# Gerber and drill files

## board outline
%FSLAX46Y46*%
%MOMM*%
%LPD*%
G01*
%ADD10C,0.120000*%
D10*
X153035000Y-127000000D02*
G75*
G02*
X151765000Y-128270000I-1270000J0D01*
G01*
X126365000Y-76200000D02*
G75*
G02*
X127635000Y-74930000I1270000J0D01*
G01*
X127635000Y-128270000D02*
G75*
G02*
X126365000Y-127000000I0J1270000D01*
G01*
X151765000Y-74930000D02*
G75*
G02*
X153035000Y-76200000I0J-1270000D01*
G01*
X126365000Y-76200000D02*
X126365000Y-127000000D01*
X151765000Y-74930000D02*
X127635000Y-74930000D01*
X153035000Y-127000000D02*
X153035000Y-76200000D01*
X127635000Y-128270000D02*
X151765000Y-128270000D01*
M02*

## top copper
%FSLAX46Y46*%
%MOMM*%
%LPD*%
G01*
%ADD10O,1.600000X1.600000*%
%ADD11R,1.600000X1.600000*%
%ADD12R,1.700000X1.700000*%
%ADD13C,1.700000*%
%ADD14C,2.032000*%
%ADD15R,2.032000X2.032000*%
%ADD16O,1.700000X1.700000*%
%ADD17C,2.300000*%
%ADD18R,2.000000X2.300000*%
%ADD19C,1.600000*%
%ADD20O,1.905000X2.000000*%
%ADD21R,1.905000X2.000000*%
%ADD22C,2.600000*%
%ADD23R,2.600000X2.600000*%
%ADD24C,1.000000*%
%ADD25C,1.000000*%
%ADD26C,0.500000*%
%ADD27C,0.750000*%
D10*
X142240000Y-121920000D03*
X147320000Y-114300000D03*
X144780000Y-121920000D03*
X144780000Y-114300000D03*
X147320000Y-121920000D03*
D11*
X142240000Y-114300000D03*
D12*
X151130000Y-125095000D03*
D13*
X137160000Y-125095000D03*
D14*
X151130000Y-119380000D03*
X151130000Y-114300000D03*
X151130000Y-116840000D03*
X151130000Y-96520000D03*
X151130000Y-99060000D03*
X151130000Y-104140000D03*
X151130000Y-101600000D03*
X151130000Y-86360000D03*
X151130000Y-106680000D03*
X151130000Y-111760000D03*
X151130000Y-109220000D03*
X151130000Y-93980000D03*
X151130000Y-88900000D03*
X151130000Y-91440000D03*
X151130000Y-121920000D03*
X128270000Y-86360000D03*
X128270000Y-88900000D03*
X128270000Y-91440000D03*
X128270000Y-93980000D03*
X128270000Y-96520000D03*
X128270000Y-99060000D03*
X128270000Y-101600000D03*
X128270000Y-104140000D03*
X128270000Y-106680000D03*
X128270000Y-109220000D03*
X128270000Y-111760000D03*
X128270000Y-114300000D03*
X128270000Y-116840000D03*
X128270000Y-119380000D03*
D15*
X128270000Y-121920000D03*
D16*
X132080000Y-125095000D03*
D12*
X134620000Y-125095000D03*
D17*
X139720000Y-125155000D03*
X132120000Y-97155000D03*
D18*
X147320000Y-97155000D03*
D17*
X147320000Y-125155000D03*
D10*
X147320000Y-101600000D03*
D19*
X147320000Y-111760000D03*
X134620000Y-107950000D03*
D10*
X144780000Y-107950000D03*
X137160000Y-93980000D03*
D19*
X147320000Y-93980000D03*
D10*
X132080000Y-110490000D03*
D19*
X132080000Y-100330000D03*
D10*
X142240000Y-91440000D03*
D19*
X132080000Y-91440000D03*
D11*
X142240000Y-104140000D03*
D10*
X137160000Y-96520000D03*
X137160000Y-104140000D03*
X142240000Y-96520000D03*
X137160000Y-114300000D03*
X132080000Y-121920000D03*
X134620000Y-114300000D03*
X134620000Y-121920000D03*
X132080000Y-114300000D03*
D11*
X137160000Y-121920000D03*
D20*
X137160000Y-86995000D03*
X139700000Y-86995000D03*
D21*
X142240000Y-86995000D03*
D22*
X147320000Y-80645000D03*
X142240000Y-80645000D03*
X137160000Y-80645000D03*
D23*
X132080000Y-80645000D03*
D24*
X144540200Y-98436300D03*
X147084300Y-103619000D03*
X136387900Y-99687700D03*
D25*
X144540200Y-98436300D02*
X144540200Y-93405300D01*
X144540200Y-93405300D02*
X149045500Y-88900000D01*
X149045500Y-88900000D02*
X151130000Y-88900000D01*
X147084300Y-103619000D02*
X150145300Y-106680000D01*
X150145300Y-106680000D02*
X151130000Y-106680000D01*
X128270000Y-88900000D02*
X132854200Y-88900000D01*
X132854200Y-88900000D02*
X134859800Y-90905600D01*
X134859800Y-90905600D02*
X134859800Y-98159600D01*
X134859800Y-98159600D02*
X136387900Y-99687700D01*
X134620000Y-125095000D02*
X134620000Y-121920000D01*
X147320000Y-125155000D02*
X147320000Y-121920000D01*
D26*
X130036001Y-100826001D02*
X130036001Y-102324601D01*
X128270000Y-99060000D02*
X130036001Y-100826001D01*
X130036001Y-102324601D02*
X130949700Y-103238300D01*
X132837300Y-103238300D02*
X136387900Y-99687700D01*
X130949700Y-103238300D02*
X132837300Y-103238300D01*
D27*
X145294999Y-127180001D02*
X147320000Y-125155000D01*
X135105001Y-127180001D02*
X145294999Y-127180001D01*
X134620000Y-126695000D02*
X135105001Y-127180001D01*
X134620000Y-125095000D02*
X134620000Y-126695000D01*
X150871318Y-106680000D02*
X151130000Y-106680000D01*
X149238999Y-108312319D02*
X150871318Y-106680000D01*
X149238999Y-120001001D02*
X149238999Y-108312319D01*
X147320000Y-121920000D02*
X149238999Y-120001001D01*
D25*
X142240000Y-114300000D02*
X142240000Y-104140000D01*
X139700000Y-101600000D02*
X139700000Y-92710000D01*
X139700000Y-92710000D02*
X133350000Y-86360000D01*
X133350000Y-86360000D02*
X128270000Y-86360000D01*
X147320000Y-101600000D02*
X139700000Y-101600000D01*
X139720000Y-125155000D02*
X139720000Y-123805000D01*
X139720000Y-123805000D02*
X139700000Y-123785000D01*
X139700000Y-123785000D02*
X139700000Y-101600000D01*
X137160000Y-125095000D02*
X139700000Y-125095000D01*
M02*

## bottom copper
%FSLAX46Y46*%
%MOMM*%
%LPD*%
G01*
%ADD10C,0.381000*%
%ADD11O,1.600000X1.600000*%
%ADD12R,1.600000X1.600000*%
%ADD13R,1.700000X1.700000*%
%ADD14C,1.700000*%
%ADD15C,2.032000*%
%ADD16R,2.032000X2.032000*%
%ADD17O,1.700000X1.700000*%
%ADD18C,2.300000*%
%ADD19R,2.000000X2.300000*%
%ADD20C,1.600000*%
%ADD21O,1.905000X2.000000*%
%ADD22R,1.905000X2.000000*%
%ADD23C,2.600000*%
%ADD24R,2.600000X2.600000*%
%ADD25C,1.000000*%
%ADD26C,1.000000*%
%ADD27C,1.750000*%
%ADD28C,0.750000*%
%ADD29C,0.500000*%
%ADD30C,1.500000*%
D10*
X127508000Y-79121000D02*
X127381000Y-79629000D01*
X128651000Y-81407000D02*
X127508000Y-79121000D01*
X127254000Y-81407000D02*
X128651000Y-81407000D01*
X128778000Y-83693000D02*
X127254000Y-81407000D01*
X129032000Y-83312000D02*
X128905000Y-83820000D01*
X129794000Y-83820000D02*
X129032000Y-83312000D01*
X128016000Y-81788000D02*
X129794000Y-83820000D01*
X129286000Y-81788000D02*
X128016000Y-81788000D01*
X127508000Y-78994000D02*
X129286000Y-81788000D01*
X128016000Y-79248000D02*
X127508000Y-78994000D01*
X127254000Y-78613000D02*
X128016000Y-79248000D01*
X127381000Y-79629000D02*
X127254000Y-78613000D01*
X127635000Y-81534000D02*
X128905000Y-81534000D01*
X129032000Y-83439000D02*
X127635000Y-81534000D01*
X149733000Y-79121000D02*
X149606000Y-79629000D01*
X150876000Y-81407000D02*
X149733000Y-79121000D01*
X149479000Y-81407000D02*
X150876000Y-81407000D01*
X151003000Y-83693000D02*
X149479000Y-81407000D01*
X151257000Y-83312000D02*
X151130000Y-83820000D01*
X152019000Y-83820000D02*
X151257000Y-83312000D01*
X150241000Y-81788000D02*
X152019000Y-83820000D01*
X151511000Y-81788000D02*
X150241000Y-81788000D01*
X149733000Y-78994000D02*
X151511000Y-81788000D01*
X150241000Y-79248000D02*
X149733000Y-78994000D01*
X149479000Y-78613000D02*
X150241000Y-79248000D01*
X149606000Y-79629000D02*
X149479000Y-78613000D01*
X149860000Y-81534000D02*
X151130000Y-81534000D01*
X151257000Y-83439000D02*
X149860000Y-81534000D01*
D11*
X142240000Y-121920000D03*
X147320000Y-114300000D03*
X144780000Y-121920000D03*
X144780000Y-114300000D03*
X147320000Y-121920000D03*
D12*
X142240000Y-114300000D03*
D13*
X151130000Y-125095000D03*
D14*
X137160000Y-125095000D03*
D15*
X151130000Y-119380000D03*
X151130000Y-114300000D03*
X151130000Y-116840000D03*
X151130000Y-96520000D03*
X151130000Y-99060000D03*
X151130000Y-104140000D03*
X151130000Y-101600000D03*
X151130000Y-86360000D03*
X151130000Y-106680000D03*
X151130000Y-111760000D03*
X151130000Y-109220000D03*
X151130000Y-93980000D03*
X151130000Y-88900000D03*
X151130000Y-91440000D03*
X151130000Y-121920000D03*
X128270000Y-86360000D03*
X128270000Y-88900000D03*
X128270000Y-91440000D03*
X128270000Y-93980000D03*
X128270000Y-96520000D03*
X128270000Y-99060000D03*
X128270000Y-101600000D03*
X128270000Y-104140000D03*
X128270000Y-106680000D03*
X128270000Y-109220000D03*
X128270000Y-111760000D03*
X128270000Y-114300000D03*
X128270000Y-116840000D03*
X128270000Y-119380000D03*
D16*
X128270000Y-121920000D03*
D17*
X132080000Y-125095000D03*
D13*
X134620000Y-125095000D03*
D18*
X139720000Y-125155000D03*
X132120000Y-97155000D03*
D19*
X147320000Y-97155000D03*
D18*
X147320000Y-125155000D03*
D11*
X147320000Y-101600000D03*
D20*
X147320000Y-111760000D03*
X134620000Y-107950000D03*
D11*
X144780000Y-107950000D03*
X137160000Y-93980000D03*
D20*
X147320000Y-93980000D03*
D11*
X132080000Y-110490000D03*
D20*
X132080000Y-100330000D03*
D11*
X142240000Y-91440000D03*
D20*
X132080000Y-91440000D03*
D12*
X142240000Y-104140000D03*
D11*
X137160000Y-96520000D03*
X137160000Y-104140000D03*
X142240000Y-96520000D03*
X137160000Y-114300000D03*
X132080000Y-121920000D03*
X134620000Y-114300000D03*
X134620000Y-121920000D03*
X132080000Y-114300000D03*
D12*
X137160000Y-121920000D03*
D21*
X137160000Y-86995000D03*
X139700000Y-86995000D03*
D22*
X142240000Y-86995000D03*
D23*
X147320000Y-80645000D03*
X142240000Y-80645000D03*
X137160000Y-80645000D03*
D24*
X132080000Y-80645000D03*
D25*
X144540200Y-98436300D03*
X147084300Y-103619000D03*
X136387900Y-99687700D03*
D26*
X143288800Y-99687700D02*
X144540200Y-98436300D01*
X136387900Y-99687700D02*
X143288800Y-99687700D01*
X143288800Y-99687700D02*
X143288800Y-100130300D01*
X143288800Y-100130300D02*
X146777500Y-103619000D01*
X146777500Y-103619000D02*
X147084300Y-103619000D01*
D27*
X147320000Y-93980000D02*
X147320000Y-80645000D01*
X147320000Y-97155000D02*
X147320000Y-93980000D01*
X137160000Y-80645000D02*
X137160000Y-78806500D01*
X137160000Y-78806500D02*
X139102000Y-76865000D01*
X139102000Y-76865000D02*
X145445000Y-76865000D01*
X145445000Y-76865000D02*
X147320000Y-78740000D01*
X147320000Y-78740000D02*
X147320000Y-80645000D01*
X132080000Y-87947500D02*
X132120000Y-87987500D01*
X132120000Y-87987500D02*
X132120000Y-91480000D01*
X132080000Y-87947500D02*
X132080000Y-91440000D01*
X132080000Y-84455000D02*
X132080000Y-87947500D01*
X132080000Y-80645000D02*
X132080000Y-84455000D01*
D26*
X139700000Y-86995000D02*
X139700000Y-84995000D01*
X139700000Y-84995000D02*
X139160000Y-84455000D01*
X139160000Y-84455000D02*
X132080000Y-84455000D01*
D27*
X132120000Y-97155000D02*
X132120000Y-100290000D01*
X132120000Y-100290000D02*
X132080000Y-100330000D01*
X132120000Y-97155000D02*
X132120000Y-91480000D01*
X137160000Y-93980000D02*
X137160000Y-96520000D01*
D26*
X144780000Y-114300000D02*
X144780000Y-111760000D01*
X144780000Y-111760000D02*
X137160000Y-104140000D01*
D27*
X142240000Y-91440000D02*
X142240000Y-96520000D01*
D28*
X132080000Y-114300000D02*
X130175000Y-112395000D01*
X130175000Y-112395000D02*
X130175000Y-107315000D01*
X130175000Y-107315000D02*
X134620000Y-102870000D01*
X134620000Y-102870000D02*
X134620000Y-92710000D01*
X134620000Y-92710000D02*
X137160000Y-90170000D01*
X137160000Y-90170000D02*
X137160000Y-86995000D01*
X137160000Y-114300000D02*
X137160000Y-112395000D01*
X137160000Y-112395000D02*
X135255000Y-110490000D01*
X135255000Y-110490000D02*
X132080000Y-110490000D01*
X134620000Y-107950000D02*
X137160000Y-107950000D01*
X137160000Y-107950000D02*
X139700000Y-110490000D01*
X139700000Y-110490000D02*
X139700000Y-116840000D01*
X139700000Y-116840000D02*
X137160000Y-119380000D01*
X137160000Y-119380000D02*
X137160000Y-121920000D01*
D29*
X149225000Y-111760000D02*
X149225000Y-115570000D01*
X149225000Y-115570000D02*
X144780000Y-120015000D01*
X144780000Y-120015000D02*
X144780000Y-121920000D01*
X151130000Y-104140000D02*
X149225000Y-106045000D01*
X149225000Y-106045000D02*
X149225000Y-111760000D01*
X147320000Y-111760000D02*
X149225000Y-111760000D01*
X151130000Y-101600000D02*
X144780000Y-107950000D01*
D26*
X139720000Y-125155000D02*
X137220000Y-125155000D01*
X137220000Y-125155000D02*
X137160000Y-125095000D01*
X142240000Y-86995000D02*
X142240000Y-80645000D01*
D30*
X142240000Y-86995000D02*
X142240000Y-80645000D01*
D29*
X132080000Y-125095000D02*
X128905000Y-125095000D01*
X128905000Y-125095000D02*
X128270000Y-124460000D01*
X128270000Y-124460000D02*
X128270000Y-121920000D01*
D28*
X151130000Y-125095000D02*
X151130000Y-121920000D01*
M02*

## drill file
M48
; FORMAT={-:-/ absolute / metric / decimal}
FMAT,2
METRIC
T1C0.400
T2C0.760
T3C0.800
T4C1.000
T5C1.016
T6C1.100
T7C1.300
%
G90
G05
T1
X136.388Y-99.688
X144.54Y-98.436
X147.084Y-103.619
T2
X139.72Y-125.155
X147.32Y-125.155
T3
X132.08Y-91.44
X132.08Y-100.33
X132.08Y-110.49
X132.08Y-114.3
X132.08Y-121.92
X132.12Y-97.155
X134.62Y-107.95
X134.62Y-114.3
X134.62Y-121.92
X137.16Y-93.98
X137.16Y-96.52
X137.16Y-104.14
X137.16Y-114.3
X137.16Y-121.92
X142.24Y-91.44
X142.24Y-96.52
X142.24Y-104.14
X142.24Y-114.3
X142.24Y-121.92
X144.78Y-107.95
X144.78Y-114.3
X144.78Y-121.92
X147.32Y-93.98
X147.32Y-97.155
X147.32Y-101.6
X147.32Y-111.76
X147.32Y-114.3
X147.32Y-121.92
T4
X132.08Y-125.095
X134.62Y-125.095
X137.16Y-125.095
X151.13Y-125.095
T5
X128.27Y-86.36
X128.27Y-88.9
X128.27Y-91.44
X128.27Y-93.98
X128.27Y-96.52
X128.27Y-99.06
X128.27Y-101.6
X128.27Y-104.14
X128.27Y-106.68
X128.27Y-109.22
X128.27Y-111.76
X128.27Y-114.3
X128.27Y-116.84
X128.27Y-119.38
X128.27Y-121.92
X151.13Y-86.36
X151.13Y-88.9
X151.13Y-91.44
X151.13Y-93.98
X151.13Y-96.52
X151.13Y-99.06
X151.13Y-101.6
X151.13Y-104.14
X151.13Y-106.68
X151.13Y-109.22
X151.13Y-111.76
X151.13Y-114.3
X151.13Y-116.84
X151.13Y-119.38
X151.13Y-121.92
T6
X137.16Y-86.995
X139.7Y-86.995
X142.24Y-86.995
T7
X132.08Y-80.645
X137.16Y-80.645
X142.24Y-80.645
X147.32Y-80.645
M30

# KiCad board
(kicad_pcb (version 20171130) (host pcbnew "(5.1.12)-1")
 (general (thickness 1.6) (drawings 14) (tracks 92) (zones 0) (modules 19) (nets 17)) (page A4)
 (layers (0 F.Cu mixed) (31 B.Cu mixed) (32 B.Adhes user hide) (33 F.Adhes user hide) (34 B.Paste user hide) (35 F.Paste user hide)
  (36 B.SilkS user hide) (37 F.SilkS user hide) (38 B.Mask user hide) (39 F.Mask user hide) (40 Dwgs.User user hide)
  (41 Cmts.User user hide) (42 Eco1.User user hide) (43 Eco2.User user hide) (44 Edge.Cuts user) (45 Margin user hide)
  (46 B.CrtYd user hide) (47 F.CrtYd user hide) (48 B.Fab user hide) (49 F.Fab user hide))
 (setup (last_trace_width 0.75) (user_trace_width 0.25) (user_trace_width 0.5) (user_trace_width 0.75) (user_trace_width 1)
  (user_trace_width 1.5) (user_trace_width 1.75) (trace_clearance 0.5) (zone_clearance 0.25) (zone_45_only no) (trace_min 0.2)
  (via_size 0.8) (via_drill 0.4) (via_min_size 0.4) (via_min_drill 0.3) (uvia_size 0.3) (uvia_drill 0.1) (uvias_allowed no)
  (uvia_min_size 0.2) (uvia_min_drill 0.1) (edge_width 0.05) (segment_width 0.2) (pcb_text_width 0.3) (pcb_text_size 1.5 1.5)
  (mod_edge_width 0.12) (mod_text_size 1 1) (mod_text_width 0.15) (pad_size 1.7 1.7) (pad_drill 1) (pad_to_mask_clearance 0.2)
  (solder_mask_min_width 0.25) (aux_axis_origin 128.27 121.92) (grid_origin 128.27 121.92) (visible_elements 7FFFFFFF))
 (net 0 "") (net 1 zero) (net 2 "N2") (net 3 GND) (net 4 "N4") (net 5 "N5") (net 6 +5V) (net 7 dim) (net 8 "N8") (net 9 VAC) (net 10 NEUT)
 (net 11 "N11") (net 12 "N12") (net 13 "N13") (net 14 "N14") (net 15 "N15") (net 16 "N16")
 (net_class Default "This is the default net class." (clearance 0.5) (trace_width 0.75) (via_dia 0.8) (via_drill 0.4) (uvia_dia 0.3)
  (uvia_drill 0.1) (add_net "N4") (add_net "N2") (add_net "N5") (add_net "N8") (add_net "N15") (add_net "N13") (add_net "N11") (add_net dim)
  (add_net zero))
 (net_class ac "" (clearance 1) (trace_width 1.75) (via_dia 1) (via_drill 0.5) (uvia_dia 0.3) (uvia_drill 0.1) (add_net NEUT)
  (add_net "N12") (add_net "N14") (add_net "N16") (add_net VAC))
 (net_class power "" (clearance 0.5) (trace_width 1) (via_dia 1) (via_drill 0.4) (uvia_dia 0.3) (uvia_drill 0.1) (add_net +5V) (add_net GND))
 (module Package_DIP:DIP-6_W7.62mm (layer B.Cu) (at 142.24 114.3 270)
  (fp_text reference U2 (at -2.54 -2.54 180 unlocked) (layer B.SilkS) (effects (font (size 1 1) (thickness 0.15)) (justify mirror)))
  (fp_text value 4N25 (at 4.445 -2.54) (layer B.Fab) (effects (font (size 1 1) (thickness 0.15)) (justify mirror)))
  (pad 6 thru_hole oval (at 7.62 0 270) (size 1.6 1.6) (drill 0.8) (layers *.Cu *.Mask))
  (pad 3 thru_hole oval (at 0 -5.08 270) (size 1.6 1.6) (drill 0.8) (layers *.Cu *.Mask))
  (pad 5 thru_hole oval (at 7.62 -2.54 270) (size 1.6 1.6) (drill 0.8) (layers *.Cu *.Mask) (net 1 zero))
  (pad 2 thru_hole oval (at 0 -2.54 270) (size 1.6 1.6) (drill 0.8) (layers *.Cu *.Mask) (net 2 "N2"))
  (pad 4 thru_hole oval (at 7.62 -5.08 270) (size 1.6 1.6) (drill 0.8) (layers *.Cu *.Mask) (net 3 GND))
  (pad 1 thru_hole rect (at 0 0 270) (size 1.6 1.6) (drill 0.8) (layers *.Cu *.Mask) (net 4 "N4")))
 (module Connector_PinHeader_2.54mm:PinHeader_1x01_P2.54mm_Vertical (layer B.Cu) (at 151.13 125.095)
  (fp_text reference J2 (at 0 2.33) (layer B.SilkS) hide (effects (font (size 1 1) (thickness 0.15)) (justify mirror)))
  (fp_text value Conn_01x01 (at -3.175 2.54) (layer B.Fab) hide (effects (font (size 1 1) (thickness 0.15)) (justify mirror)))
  (pad 1 thru_hole rect (at 0 0) (size 1.7 1.7) (drill 1) (layers *.Cu *.Mask) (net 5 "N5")))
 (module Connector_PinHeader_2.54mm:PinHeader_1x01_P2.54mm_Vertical (layer B.Cu) (at 137.16 125.095)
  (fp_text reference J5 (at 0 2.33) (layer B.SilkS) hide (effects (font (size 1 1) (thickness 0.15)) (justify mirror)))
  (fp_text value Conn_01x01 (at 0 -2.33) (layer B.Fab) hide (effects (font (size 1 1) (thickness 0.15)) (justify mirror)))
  (pad 1 thru_hole circle (at 0 0) (size 1.7 1.7) (drill 1) (layers *.Cu *.Mask) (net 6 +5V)))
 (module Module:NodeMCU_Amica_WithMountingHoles (layer B.Cu) (at 128.27 121.92)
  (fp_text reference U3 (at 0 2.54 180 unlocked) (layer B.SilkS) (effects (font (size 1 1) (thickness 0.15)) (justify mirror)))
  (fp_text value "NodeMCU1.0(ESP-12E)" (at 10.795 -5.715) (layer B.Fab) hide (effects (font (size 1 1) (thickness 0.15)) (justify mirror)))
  (pad 29 thru_hole circle (at 22.86 -2.54) (size 2.032 2.032) (drill 1.016) (layers *.Cu *.Mask))
  (pad 27 thru_hole circle (at 22.86 -7.62) (size 2.032 2.032) (drill 1.016) (layers *.Cu *.Mask))
  (pad 28 thru_hole circle (at 22.86 -5.08) (size 2.032 2.032) (drill 1.016) (layers *.Cu *.Mask))
  (pad 20 thru_hole circle (at 22.86 -25.4) (size 2.032 2.032) (drill 1.016) (layers *.Cu *.Mask))
  (pad 21 thru_hole circle (at 22.86 -22.86) (size 2.032 2.032) (drill 1.016) (layers *.Cu *.Mask))
  (pad 23 thru_hole circle (at 22.86 -17.78) (size 2.032 2.032) (drill 1.016) (layers *.Cu *.Mask) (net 1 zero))
  (pad 22 thru_hole circle (at 22.86 -20.32) (size 2.032 2.032) (drill 1.016) (layers *.Cu *.Mask) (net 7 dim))
  (pad 16 thru_hole circle (at 22.86 -35.56) (size 2.032 2.032) (drill 1.016) (layers *.Cu *.Mask))
  (pad 24 thru_hole circle (at 22.86 -15.24) (size 2.032 2.032) (drill 1.016) (layers *.Cu *.Mask) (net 3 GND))
  (pad 26 thru_hole circle (at 22.86 -10.16) (size 2.032 2.032) (drill 1.016) (layers *.Cu *.Mask))
  (pad 25 thru_hole circle (at 22.86 -12.7) (size 2.032 2.032) (drill 1.016) (layers *.Cu *.Mask))
  (pad 19 thru_hole circle (at 22.86 -27.94) (size 2.032 2.032) (drill 1.016) (layers *.Cu *.Mask))
  (pad 17 thru_hole circle (at 22.86 -33.02) (size 2.032 2.032) (drill 1.016) (layers *.Cu *.Mask) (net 3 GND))
  (pad 18 thru_hole circle (at 22.86 -30.48) (size 2.032 2.032) (drill 1.016) (layers *.Cu *.Mask))
  (pad 30 thru_hole circle (at 22.86 0) (size 2.032 2.032) (drill 1.016) (layers *.Cu *.Mask) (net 5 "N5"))
  (pad 15 thru_hole circle (at 0 -35.56) (size 2.032 2.032) (drill 1.016) (layers *.Cu *.Mask) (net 6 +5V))
  (pad 14 thru_hole circle (at 0 -33.02) (size 2.032 2.032) (drill 1.016) (layers *.Cu *.Mask) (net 3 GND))
  (pad 13 thru_hole circle (at 0 -30.48) (size 2.032 2.032) (drill 1.016) (layers *.Cu *.Mask))
  (pad 12 thru_hole circle (at 0 -27.94) (size 2.032 2.032) (drill 1.016) (layers *.Cu *.Mask))
  (pad 11 thru_hole circle (at 0 -25.4) (size 2.032 2.032) (drill 1.016) (layers *.Cu *.Mask))
  (pad 10 thru_hole circle (at 0 -22.86) (size 2.032 2.032) (drill 1.016) (layers *.Cu *.Mask) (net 3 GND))
  (pad 9 thru_hole circle (at 0 -20.32) (size 2.032 2.032) (drill 1.016) (layers *.Cu *.Mask))
  (pad 8 thru_hole circle (at 0 -17.78) (size 2.032 2.032) (drill 1.016) (layers *.Cu *.Mask))
  (pad 7 thru_hole circle (at 0 -15.24) (size 2.032 2.032) (drill 1.016) (layers *.Cu *.Mask))
  (pad 6 thru_hole circle (at 0 -12.7) (size 2.032 2.032) (drill 1.016) (layers *.Cu *.Mask))
  (pad 5 thru_hole circle (at 0 -10.16) (size 2.032 2.032) (drill 1.016) (layers *.Cu *.Mask))
  (pad 4 thru_hole circle (at 0 -7.62) (size 2.032 2.032) (drill 1.016) (layers *.Cu *.Mask))
  (pad 3 thru_hole circle (at 0 -5.08) (size 2.032 2.032) (drill 1.016) (layers *.Cu *.Mask))
  (pad 2 thru_hole circle (at 0 -2.54) (size 2.032 2.032) (drill 1.016) (layers *.Cu *.Mask))
  (pad 1 thru_hole rect (at 0 0) (size 2.032 2.032) (drill 1.016) (layers *.Cu *.Mask) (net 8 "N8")))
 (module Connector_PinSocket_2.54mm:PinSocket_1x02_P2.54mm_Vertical (layer B.Cu) (at 134.62 125.095 90)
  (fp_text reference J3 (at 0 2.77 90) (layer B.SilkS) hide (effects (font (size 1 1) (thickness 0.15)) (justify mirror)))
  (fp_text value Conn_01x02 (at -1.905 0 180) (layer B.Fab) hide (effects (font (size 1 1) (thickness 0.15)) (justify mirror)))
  (pad 2 thru_hole oval (at 0 -2.54 90) (size 1.7 1.7) (drill 1) (layers *.Cu *.Mask) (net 8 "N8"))
  (pad 1 thru_hole rect (at 0 0 90) (size 1.7 1.7) (drill 1) (layers *.Cu *.Mask) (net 3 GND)))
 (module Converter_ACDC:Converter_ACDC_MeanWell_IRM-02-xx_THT (layer F.Cu) (at 147.32 97.155 270)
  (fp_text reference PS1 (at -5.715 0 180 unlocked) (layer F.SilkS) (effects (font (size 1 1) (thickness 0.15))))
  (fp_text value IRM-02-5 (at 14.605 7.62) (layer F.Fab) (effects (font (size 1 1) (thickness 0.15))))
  (pad 4 thru_hole circle (at 28 7.6 270) (size 2.3 2.3) (drill 0.76) (layers *.Cu *.Mask) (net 6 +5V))
  (pad 2 thru_hole circle (at 0 15.2 270) (size 2.3 2.3) (drill 0.8) (layers *.Cu *.Mask) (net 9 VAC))
  (pad 1 thru_hole rect (at 0 0 270) (size 2.3 2) (drill 0.8) (layers *.Cu *.Mask) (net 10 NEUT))
  (pad 3 thru_hole circle (at 28 0 270) (size 2.3 2.3) (drill 0.76) (layers *.Cu *.Mask) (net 3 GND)))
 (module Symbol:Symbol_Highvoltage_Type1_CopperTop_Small (layer B.Cu) (at 127.635 80.645)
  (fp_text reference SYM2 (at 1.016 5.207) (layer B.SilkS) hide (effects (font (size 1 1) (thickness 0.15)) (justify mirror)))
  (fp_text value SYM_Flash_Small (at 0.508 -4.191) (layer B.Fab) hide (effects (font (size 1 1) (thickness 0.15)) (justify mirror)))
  (fp_line (start -0.127 -1.524) (end -0.254 -1.016) (layer B.Cu) (width 0.381))
  (fp_line (start 1.016 0.762) (end -0.127 -1.524) (layer B.Cu) (width 0.381))
  (fp_line (start -0.381 0.762) (end 1.016 0.762) (layer B.Cu) (width 0.381))
  (fp_line (start 1.143 3.048) (end -0.381 0.762) (layer B.Cu) (width 0.381))
  (fp_line (start 1.397 2.667) (end 1.27 3.175) (layer B.Cu) (width 0.381))
  (fp_line (start 2.159 3.175) (end 1.397 2.667) (layer B.Cu) (width 0.381))
  (fp_line (start 0.381 1.143) (end 2.159 3.175) (layer B.Cu) (width 0.381))
  (fp_line (start 1.651 1.143) (end 0.381 1.143) (layer B.Cu) (width 0.381))
  (fp_line (start -0.127 -1.651) (end 1.651 1.143) (layer B.Cu) (width 0.381))
  (fp_line (start 0.381 -1.397) (end -0.127 -1.651) (layer B.Cu) (width 0.381))
  (fp_line (start -0.381 -2.032) (end 0.381 -1.397) (layer B.Cu) (width 0.381))
  (fp_line (start -0.254 -1.016) (end -0.381 -2.032) (layer B.Cu) (width 0.381))
  (fp_line (start 0 0.889) (end 1.27 0.889) (layer B.Cu) (width 0.381))
  (fp_line (start 1.397 2.794) (end 0 0.889) (layer B.Cu) (width 0.381)))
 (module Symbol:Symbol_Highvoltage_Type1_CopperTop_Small (layer B.Cu) (at 149.86 80.645)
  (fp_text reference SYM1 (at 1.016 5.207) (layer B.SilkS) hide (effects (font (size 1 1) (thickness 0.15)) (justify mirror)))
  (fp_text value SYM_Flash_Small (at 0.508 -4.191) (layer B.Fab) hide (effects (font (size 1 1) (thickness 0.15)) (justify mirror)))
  (fp_line (start -0.127 -1.524) (end -0.254 -1.016) (layer B.Cu) (width 0.381))
  (fp_line (start 1.016 0.762) (end -0.127 -1.524) (layer B.Cu) (width 0.381))
  (fp_line (start -0.381 0.762) (end 1.016 0.762) (layer B.Cu) (width 0.381))
  (fp_line (start 1.143 3.048) (end -0.381 0.762) (layer B.Cu) (width 0.381))
  (fp_line (start 1.397 2.667) (end 1.27 3.175) (layer B.Cu) (width 0.381))
  (fp_line (start 2.159 3.175) (end 1.397 2.667) (layer B.Cu) (width 0.381))
  (fp_line (start 0.381 1.143) (end 2.159 3.175) (layer B.Cu) (width 0.381))
  (fp_line (start 1.651 1.143) (end 0.381 1.143) (layer B.Cu) (width 0.381))
  (fp_line (start -0.127 -1.651) (end 1.651 1.143) (layer B.Cu) (width 0.381))
  (fp_line (start 0.381 -1.397) (end -0.127 -1.651) (layer B.Cu) (width 0.381))
  (fp_line (start -0.381 -2.032) (end 0.381 -1.397) (layer B.Cu) (width 0.381))
  (fp_line (start -0.254 -1.016) (end -0.381 -2.032) (layer B.Cu) (width 0.381))
  (fp_line (start 0 0.889) (end 1.27 0.889) (layer B.Cu) (width 0.381))
  (fp_line (start 1.397 2.794) (end 0 0.889) (layer B.Cu) (width 0.381)))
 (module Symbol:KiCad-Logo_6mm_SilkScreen (layer F.Cu) (at 143.51 105.41 90)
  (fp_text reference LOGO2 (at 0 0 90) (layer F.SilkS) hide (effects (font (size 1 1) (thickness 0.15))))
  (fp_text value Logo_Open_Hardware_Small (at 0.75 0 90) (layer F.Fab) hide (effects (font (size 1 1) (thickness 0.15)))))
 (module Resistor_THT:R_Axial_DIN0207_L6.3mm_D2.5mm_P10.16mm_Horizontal (layer B.Cu) (at 147.32 111.76 90)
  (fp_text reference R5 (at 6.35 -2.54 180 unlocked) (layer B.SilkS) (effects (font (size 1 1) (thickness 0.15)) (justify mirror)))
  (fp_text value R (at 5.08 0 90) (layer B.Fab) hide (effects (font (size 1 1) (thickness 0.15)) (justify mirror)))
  (pad 2 thru_hole oval (at 10.16 0 90) (size 1.6 1.6) (drill 0.8) (layers *.Cu *.Mask) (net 6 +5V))
  (pad 1 thru_hole circle (at 0 0 90) (size 1.6 1.6) (drill 0.8) (layers *.Cu *.Mask) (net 1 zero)))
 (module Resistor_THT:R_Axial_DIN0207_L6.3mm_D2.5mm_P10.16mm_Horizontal (layer B.Cu) (at 134.62 107.95)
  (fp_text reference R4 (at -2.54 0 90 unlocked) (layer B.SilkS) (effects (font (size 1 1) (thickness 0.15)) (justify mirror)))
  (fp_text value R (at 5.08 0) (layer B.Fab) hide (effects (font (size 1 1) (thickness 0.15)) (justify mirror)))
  (pad 1 thru_hole circle (at 0 0) (size 1.6 1.6) (drill 0.8) (layers *.Cu *.Mask) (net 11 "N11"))
  (pad 2 thru_hole oval (at 10.16 0) (size 1.6 1.6) (drill 0.8) (layers *.Cu *.Mask) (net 7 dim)))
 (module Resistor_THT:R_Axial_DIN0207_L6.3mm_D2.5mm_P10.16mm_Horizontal (layer B.Cu) (at 147.32 93.98 180)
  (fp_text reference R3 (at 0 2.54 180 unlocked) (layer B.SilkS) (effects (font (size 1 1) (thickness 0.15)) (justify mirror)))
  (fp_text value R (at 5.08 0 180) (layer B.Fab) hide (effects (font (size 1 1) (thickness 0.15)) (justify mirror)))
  (pad 2 thru_hole oval (at 10.16 0 180) (size 1.6 1.6) (drill 0.8) (layers *.Cu *.Mask) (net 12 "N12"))
  (pad 1 thru_hole circle (at 0 0 180) (size 1.6 1.6) (drill 0.8) (layers *.Cu *.Mask) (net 10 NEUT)))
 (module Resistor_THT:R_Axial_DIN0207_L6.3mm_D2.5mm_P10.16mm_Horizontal (layer B.Cu) (at 132.08 100.33 270)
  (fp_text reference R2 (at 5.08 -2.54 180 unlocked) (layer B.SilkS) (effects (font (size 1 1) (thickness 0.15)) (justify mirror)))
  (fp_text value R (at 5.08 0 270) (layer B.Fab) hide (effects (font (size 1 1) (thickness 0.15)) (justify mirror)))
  (pad 2 thru_hole oval (at 10.16 0 270) (size 1.6 1.6) (drill 0.8) (layers *.Cu *.Mask) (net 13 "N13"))
  (pad 1 thru_hole circle (at 0 0 270) (size 1.6 1.6) (drill 0.8) (layers *.Cu *.Mask) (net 9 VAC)))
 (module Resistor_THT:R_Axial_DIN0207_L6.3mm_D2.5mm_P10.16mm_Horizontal (layer B.Cu) (at 132.08 91.44)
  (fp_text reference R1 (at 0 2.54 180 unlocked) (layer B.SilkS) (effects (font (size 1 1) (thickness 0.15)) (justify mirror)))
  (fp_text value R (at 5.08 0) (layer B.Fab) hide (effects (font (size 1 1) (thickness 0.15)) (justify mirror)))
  (pad 2 thru_hole oval (at 10.16 0) (size 1.6 1.6) (drill 0.8) (layers *.Cu *.Mask) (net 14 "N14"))
  (pad 1 thru_hole circle (at 0 0) (size 1.6 1.6) (drill 0.8) (layers *.Cu *.Mask) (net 9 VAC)))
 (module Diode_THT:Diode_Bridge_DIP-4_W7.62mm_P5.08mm (layer B.Cu) (at 142.24 104.14 90)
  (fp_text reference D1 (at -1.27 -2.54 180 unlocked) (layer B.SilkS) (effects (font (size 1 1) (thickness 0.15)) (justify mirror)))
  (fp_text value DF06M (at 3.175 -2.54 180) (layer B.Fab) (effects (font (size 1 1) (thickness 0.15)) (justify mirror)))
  (pad 1 thru_hole rect (at 0 0 90) (size 1.6 1.6) (drill 0.8) (layers *.Cu *.Mask) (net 4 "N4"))
  (pad 3 thru_hole oval (at 7.62 -5.08 90) (size 1.6 1.6) (drill 0.8) (layers *.Cu *.Mask) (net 12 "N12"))
  (pad 2 thru_hole oval (at 0 -5.08 90) (size 1.6 1.6) (drill 0.8) (layers *.Cu *.Mask) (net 2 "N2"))
  (pad 4 thru_hole oval (at 7.62 0 90) (size 1.6 1.6) (drill 0.8) (layers *.Cu *.Mask) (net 14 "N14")))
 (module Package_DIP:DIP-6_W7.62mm (layer B.Cu) (at 137.16 121.92 90)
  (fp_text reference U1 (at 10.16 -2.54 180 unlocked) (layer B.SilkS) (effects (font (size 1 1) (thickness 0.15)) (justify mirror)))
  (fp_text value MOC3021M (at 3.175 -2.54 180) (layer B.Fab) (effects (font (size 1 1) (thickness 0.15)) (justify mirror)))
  (pad 6 thru_hole oval (at 7.62 0 90) (size 1.6 1.6) (drill 0.8) (layers *.Cu *.Mask) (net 13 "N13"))
  (pad 3 thru_hole oval (at 0 -5.08 90) (size 1.6 1.6) (drill 0.8) (layers *.Cu *.Mask))
  (pad 5 thru_hole oval (at 7.62 -2.54 90) (size 1.6 1.6) (drill 0.8) (layers *.Cu *.Mask))
  (pad 2 thru_hole oval (at 0 -2.54 90) (size 1.6 1.6) (drill 0.8) (layers *.Cu *.Mask) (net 3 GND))
  (pad 4 thru_hole oval (at 7.62 -5.08 90) (size 1.6 1.6) (drill 0.8) (layers *.Cu *.Mask) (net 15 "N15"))
  (pad 1 thru_hole rect (at 0 0 90) (size 1.6 1.6) (drill 0.8) (layers *.Cu *.Mask) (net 11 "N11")))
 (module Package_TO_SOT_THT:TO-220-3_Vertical (layer F.Cu) (at 142.24 86.995 180)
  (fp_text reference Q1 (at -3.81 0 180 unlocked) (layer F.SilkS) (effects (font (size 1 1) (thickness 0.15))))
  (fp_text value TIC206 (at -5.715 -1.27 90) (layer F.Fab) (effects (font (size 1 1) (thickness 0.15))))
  (pad 3 thru_hole oval (at 5.08 0 180) (size 1.905 2) (drill 1.1) (layers *.Cu *.Mask) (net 15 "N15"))
  (pad 2 thru_hole oval (at 2.54 0 180) (size 1.905 2) (drill 1.1) (layers *.Cu *.Mask) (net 9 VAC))
  (pad 1 thru_hole rect (at 0 0 180) (size 1.905 2) (drill 1.1) (layers *.Cu *.Mask) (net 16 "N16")))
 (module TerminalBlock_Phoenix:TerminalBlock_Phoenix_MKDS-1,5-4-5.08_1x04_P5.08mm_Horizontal (layer F.Cu) (at 132.08 80.645)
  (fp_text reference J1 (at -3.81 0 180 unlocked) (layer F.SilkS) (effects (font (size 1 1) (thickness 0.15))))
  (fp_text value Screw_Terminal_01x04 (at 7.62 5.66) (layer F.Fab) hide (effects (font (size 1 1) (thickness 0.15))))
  (pad 4 thru_hole circle (at 15.24 0) (size 2.6 2.6) (drill 1.3) (layers *.Cu *.Mask) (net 10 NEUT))
  (pad 3 thru_hole circle (at 10.16 0) (size 2.6 2.6) (drill 1.3) (layers *.Cu *.Mask) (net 16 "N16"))
  (pad 2 thru_hole circle (at 5.08 0) (size 2.6 2.6) (drill 1.3) (layers *.Cu *.Mask) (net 10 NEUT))
  (pad 1 thru_hole rect (at 0 0) (size 2.6 2.6) (drill 1.3) (layers *.Cu *.Mask) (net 9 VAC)))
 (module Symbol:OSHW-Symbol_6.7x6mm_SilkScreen (layer F.Cu) (at 143.51 118.11 90)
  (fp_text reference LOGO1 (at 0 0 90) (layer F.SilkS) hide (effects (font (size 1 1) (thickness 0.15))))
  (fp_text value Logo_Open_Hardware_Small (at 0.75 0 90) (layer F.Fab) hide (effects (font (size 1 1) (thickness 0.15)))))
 (gr_arc (start 151.765 127) (end 151.765 128.27) (angle -90) (layer Edge.Cuts) (width 0.12))
 (gr_arc (start 127.635 76.2) (end 127.635 74.93) (angle -90) (layer Edge.Cuts) (width 0.12))
 (gr_arc (start 127.635 127) (end 126.365 127) (angle -90) (layer Edge.Cuts) (width 0.12))
 (gr_arc (start 151.765 76.2) (end 153.035 76.2) (angle -90) (layer Edge.Cuts) (width 0.12))
 (gr_line (start 126.365 76.2) (end 126.365 127) (layer Edge.Cuts) (width 0.12))
 (gr_line (start 151.765 74.93) (end 127.635 74.93) (layer Edge.Cuts) (width 0.12))
 (gr_line (start 153.035 127) (end 153.035 76.2) (layer Edge.Cuts) (width 0.12))
 (gr_line (start 127.635 128.27) (end 151.765 128.27) (layer Edge.Cuts) (width 0.12))
 (segment (start 143.2888 99.6877) (end 144.5402 98.4363) (width 1) (layer B.Cu) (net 3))
 (segment (start 136.3879 99.6877) (end 143.2888 99.6877) (width 1) (layer B.Cu) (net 3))
 (segment (start 143.2888 99.6877) (end 143.2888 100.1303) (width 1) (layer B.Cu) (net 3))
 (segment (start 143.2888 100.1303) (end 146.7775 103.619) (width 1) (layer B.Cu) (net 3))
 (segment (start 146.7775 103.619) (end 147.0843 103.619) (width 1) (layer B.Cu) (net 3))
 (segment (start 144.5402 98.4363) (end 144.5402 93.4053) (width 1) (layer F.Cu) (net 3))
 (segment (start 144.5402 93.4053) (end 149.0455 88.9) (width 1) (layer F.Cu) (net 3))
 (segment (start 149.0455 88.9) (end 151.13 88.9) (width 1) (layer F.Cu) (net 3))
 (segment (start 147.0843 103.619) (end 150.1453 106.68) (width 1) (layer F.Cu) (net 3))
 (segment (start 150.1453 106.68) (end 151.13 106.68) (width 1) (layer F.Cu) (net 3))
 (segment (start 128.27 88.9) (end 132.8542 88.9) (width 1) (layer F.Cu) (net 3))
 (segment (start 132.8542 88.9) (end 134.8598 90.9056) (width 1) (layer F.Cu) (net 3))
 (segment (start 134.8598 90.9056) (end 134.8598 98.1596) (width 1) (layer F.Cu) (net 3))
 (segment (start 134.8598 98.1596) (end 136.3879 99.6877) (width 1) (layer F.Cu) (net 3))
 (segment (start 134.62 125.095) (end 134.62 121.92) (width 1) (layer F.Cu) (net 3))
 (segment (start 147.32 125.155) (end 147.32 121.92) (width 1) (layer F.Cu) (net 3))
 (via (at 144.5402 98.4363) (size 1) (layers F.Cu B.Cu) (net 3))
 (via (at 147.0843 103.619) (size 1) (layers F.Cu B.Cu) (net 3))
 (via (at 136.3879 99.6877) (size 1) (layers F.Cu B.Cu) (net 3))
 (segment (start 130.036001 100.826001) (end 130.036001 102.324601) (width 0.5) (layer F.Cu) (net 3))
 (segment (start 128.27 99.06) (end 130.036001 100.826001) (width 0.5) (layer F.Cu) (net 3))
 (segment (start 130.036001 102.324601) (end 130.9497 103.2383) (width 0.5) (layer F.Cu) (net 3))
 (segment (start 132.8373 103.2383) (end 136.3879 99.6877) (width 0.5) (layer F.Cu) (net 3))
 (segment (start 130.9497 103.2383) (end 132.8373 103.2383) (width 0.5) (layer F.Cu) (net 3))
 (segment (start 145.294999 127.180001) (end 147.32 125.155) (width 0.75) (layer F.Cu) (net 3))
 (segment (start 135.105001 127.180001) (end 145.294999 127.180001) (width 0.75) (layer F.Cu) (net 3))
 (segment (start 134.62 126.695) (end 135.105001 127.180001) (width 0.75) (layer F.Cu) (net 3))
 (segment (start 134.62 125.095) (end 134.62 126.695) (width 0.75) (layer F.Cu) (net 3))
 (segment (start 150.871318 106.68) (end 151.13 106.68) (width 0.75) (layer F.Cu) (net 3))
 (segment (start 149.238999 108.312319) (end 150.871318 106.68) (width 0.75) (layer F.Cu) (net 3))
 (segment (start 149.238999 120.001001) (end 149.238999 108.312319) (width 0.75) (layer F.Cu) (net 3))
 (segment (start 147.32 121.92) (end 149.238999 120.001001) (width 0.75) (layer F.Cu) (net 3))
 (segment (start 147.32 93.98) (end 147.32 80.645) (width 1.75) (layer B.Cu) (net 10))
 (segment (start 147.32 97.155) (end 147.32 93.98) (width 1.75) (layer B.Cu) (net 10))
 (segment (start 137.16 80.645) (end 137.16 78.8065) (width 1.75) (layer B.Cu) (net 10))
 (segment (start 137.16 78.8065) (end 139.102 76.865) (width 1.75) (layer B.Cu) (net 10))
 (segment (start 139.102 76.865) (end 145.445 76.865) (width 1.75) (layer B.Cu) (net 10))
 (segment (start 145.445 76.865) (end 147.32 78.74) (width 1.75) (layer B.Cu) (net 10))
 (segment (start 147.32 78.74) (end 147.32 80.645) (width 1.75) (layer B.Cu) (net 10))
 (segment (start 132.08 87.9475) (end 132.12 87.9875) (width 1.75) (layer B.Cu) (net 9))
 (segment (start 132.12 87.9875) (end 132.12 91.48) (width 1.75) (layer B.Cu) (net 9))
 (segment (start 132.08 87.9475) (end 132.08 91.44) (width 1.75) (layer B.Cu) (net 9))
 (segment (start 132.08 84.455) (end 132.08 87.9475) (width 1.75) (layer B.Cu) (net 9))
 (segment (start 132.08 80.645) (end 132.08 84.455) (width 1.75) (layer B.Cu) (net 9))
 (segment (start 139.7 86.995) (end 139.7 84.995) (width 1) (layer B.Cu) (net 9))
 (segment (start 139.7 84.995) (end 139.16 84.455) (width 1) (layer B.Cu) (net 9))
 (segment (start 139.16 84.455) (end 132.08 84.455) (width 1) (layer B.Cu) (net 9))
 (segment (start 132.12 97.155) (end 132.12 100.29) (width 1.75) (layer B.Cu) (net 9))
 (segment (start 132.12 100.29) (end 132.08 100.33) (width 1.75) (layer B.Cu) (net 9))
 (segment (start 132.12 97.155) (end 132.12 91.48) (width 1.75) (layer B.Cu) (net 9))
 (segment (start 142.24 114.3) (end 142.24 104.14) (width 1) (layer F.Cu) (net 4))
 (segment (start 137.16 93.98) (end 137.16 96.52) (width 1.75) (layer B.Cu) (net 12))
 (segment (start 144.78 114.3) (end 144.78 111.76) (width 1) (layer B.Cu) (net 2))
 (segment (start 144.78 111.76) (end 137.16 104.14) (width 1) (layer B.Cu) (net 2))
 (segment (start 142.24 91.44) (end 142.24 96.52) (width 1.75) (layer B.Cu) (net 14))
 (segment (start 132.08 114.3) (end 130.175 112.395) (width 0.75) (layer B.Cu) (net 15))
 (segment (start 130.175 112.395) (end 130.175 107.315) (width 0.75) (layer B.Cu) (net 15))
 (segment (start 130.175 107.315) (end 134.62 102.87) (width 0.75) (layer B.Cu) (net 15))
 (segment (start 134.62 102.87) (end 134.62 92.71) (width 0.75) (layer B.Cu) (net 15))
 (segment (start 134.62 92.71) (end 137.16 90.17) (width 0.75) (layer B.Cu) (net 15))
 (segment (start 137.16 90.17) (end 137.16 86.995) (width 0.75) (layer B.Cu) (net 15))
 (segment (start 137.16 114.3) (end 137.16 112.395) (width 0.75) (layer B.Cu) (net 13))
 (segment (start 137.16 112.395) (end 135.255 110.49) (width 0.75) (layer B.Cu) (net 13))
 (segment (start 135.255 110.49) (end 132.08 110.49) (width 0.75) (layer B.Cu) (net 13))
 (segment (start 134.62 107.95) (end 137.16 107.95) (width 0.75) (layer B.Cu) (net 11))
 (segment (start 137.16 107.95) (end 139.7 110.49) (width 0.75) (layer B.Cu) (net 11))
 (segment (start 139.7 110.49) (end 139.7 116.84) (width 0.75) (layer B.Cu) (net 11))
 (segment (start 139.7 116.84) (end 137.16 119.38) (width 0.75) (layer B.Cu) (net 11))
 (segment (start 137.16 119.38) (end 137.16 121.92) (width 0.75) (layer B.Cu) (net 11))
 (segment (start 149.225 111.76) (end 149.225 115.57) (width 0.5) (layer B.Cu) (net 1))
 (segment (start 149.225 115.57) (end 144.78 120.015) (width 0.5) (layer B.Cu) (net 1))
 (segment (start 144.78 120.015) (end 144.78 121.92) (width 0.5) (layer B.Cu) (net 1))
 (segment (start 151.13 104.14) (end 149.225 106.045) (width 0.5) (layer B.Cu) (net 1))
 (segment (start 149.225 106.045) (end 149.225 111.76) (width 0.5) (layer B.Cu) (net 1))
 (segment (start 147.32 111.76) (end 149.225 111.76) (width 0.5) (layer B.Cu) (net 1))
 (segment (start 151.13 101.6) (end 144.78 107.95) (width 0.5) (layer B.Cu) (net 7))
 (segment (start 139.72 125.155) (end 137.22 125.155) (width 1) (layer B.Cu) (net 6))
 (segment (start 137.22 125.155) (end 137.16 125.095) (width 1) (layer B.Cu) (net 6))
 (segment (start 139.7 101.6) (end 139.7 92.71) (width 1) (layer F.Cu) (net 6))
 (segment (start 139.7 92.71) (end 133.35 86.36) (width 1) (layer F.Cu) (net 6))
 (segment (start 133.35 86.36) (end 128.27 86.36) (width 1) (layer F.Cu) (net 6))
 (segment (start 147.32 101.6) (end 139.7 101.6) (width 1) (layer F.Cu) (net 6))
 (segment (start 139.72 125.155) (end 139.72 123.805) (width 1) (layer F.Cu) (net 6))
 (segment (start 139.72 123.805) (end 139.7 123.785) (width 1) (layer F.Cu) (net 6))
 (segment (start 139.7 123.785) (end 139.7 101.6) (width 1) (layer F.Cu) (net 6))
 (segment (start 137.16 125.095) (end 139.7 125.095) (width 1) (layer F.Cu) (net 6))
 (segment (start 142.24 86.995) (end 142.24 80.645) (width 1) (layer B.Cu) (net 16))
 (segment (start 142.24 86.995) (end 142.24 80.645) (width 1.5) (layer B.Cu) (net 16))
 (segment (start 132.08 125.095) (end 128.905 125.095) (width 0.5) (layer B.Cu) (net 8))
 (segment (start 128.905 125.095) (end 128.27 124.46) (width 0.5) (layer B.Cu) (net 8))
 (segment (start 128.27 124.46) (end 128.27 121.92) (width 0.5) (layer B.Cu) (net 8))
 (segment (start 151.13 125.095) (end 151.13 121.92) (width 0.75) (layer B.Cu) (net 5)))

